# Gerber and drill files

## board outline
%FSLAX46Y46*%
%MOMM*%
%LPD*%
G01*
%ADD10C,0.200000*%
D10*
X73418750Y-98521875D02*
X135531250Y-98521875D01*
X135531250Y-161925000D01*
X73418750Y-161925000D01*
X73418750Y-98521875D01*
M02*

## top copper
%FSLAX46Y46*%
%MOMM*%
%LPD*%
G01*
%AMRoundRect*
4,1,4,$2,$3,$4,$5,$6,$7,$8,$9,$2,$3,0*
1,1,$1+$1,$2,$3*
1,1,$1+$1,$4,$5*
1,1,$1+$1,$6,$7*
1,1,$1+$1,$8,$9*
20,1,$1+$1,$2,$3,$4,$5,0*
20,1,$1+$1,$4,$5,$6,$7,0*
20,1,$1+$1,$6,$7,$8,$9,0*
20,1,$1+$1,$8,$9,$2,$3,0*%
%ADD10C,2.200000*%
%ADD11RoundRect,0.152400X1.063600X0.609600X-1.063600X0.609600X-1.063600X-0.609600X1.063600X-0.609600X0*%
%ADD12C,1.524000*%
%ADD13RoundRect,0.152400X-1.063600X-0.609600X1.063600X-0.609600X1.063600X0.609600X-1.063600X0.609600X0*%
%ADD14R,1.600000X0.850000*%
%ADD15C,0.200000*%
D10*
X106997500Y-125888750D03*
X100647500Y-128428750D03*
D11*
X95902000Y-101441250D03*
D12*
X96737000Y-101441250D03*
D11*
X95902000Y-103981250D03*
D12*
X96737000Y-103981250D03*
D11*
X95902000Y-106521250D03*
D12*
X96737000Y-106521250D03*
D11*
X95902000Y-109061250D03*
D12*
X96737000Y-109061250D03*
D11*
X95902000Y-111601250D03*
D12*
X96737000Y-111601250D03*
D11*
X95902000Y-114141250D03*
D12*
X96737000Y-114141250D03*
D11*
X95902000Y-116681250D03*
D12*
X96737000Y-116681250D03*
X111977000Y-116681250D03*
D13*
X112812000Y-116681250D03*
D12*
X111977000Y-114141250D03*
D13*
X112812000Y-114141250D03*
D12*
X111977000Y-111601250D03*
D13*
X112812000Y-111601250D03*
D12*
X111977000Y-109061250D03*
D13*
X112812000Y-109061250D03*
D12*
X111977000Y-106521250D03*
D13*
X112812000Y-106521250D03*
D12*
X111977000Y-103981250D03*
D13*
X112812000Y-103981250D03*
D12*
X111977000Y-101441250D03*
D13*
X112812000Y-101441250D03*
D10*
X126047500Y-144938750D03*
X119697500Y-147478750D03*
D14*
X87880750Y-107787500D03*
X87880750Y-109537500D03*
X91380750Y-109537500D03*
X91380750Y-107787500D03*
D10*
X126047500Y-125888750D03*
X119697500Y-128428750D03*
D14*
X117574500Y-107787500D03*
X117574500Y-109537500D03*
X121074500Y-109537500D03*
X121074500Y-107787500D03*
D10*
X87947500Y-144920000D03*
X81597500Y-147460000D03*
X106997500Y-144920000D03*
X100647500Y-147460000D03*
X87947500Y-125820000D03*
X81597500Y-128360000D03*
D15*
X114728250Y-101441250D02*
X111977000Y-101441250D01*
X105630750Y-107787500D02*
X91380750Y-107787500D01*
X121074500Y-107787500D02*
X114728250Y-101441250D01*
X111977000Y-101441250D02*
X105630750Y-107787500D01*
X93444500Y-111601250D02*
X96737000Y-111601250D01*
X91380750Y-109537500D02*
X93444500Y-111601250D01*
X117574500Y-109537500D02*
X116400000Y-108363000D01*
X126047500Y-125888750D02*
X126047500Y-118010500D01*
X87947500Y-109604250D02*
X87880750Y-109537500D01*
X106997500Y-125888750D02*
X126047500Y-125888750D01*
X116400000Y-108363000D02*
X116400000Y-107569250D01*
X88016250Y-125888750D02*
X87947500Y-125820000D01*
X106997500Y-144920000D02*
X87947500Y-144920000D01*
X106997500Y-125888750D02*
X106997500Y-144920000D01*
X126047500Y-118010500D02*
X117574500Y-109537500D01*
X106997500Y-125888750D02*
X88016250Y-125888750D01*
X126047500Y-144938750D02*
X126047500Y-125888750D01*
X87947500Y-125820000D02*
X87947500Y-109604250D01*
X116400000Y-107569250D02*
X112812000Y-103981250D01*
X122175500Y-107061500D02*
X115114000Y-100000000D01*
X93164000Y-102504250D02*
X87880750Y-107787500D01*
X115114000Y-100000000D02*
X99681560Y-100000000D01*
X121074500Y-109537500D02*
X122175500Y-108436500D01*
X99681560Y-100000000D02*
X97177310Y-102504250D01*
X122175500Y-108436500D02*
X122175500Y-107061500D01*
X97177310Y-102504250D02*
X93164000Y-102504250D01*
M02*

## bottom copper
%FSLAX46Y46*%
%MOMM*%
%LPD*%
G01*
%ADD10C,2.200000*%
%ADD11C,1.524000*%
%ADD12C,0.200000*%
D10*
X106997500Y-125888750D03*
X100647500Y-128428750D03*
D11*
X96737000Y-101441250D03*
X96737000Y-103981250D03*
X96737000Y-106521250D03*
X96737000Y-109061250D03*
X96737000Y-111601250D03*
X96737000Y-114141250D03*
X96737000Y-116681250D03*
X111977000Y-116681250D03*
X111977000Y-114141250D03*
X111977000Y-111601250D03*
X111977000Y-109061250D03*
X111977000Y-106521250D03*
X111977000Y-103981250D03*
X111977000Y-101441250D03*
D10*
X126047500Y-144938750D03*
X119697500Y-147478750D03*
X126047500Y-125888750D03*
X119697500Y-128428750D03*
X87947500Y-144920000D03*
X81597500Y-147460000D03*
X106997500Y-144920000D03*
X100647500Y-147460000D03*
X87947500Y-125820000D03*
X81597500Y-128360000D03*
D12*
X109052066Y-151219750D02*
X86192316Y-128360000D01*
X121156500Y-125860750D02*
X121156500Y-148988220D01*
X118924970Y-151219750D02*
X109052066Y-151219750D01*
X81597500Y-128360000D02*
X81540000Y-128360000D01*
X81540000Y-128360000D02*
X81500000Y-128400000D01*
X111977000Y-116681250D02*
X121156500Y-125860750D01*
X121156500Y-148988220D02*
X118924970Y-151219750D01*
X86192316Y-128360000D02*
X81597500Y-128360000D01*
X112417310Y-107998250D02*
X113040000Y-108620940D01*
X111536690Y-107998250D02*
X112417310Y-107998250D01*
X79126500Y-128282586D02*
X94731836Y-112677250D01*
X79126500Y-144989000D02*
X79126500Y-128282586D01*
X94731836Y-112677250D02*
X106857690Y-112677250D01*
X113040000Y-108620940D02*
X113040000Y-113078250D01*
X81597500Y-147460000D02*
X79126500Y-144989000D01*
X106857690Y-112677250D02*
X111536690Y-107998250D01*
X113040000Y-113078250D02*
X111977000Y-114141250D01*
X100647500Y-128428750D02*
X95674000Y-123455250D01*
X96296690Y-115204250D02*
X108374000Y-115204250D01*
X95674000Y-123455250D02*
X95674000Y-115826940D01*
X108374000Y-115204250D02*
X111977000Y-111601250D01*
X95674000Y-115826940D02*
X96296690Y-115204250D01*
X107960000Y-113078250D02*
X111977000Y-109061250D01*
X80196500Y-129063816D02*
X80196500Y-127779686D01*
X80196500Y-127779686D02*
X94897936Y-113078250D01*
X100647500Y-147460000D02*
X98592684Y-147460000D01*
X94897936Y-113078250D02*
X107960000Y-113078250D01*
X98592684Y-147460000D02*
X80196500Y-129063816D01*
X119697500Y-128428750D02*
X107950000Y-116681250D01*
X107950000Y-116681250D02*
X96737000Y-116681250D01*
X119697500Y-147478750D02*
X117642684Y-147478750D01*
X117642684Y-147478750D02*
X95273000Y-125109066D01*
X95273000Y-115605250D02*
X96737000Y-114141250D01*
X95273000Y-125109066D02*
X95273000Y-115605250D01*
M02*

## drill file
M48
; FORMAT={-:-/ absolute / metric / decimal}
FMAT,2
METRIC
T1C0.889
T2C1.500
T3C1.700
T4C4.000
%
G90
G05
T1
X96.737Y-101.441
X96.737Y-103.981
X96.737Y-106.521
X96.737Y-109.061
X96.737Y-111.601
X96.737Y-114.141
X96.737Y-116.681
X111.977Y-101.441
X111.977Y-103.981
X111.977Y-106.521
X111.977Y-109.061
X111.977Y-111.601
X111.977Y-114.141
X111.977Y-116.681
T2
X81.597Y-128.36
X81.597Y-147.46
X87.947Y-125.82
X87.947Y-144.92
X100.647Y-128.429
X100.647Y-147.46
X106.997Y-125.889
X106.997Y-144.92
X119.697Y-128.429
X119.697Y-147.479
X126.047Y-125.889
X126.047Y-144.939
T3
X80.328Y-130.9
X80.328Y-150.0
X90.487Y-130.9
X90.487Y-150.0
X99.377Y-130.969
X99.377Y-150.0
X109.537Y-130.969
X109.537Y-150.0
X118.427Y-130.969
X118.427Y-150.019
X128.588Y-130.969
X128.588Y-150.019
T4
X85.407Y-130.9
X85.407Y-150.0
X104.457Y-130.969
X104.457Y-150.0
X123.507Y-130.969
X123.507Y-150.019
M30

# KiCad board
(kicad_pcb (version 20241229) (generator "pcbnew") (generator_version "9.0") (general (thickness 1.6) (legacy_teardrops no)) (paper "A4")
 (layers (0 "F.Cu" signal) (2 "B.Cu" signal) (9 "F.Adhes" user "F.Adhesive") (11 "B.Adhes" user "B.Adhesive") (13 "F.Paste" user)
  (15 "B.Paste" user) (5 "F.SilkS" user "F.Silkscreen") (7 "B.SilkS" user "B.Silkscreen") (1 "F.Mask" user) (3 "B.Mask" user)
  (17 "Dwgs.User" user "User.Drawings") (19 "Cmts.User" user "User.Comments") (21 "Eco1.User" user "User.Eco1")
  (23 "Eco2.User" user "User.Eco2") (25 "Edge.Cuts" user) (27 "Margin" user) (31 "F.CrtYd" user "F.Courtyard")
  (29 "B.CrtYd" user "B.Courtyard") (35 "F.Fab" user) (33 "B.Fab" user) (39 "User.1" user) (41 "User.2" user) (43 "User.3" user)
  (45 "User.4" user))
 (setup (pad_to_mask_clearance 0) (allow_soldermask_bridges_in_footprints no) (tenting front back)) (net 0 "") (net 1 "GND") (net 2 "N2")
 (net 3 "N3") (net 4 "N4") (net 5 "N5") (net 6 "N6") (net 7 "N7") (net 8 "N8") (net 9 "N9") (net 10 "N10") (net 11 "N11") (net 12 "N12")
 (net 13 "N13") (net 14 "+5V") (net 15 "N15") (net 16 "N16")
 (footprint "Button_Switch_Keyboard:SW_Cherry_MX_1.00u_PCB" (layer "F.Cu") (at 106.9975 125.88875)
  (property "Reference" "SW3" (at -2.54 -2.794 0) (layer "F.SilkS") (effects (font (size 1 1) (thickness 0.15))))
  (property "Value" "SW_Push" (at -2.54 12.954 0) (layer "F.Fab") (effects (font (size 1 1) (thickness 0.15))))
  (pad "" np_thru_hole circle (at -7.62 5.08) (size 1.7 1.7) (drill 1.7) (layers "*.Cu" "*.Mask"))
  (pad "" np_thru_hole circle (at -2.54 5.08) (size 4 4) (drill 4) (layers "*.Cu" "*.Mask"))
  (pad "" np_thru_hole circle (at 2.54 5.08) (size 1.7 1.7) (drill 1.7) (layers "*.Cu" "*.Mask"))
  (pad "1" thru_hole circle (at 0 0) (size 2.2 2.2) (drill 1.5) (layers "*.Cu" "*.Mask") (remove_unused_layers no) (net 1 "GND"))
  (pad "2" thru_hole circle (at -6.35 2.54) (size 2.2 2.2) (drill 1.5) (layers "*.Cu" "*.Mask") (remove_unused_layers no) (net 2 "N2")))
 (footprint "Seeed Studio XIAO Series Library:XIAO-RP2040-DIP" (layer "F.Cu") (at 104.357 109.06125)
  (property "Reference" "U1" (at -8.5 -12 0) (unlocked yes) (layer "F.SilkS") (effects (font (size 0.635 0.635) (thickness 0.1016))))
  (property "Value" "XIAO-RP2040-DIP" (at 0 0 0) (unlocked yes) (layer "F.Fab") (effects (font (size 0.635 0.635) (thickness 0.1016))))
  (pad "1" smd roundrect (at -8.455 -7.62 180) (size 2.432 1.524) (layers "F.Cu" "F.Mask") (roundrect_rratio 0.1) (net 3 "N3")
   (thermal_bridge_angle 45))
  (pad "1" thru_hole circle (at -7.62 -7.62 180) (size 1.524 1.524) (drill 0.889) (layers "*.Cu" "*.Mask") (remove_unused_layers no)
   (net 3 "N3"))
  (pad "2" smd roundrect (at -8.455 -5.08 180) (size 2.432 1.524) (layers "F.Cu" "F.Mask") (roundrect_rratio 0.1) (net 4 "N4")
   (thermal_bridge_angle 45))
  (pad "2" thru_hole circle (at -7.62 -5.08 180) (size 1.524 1.524) (drill 0.889) (layers "*.Cu" "*.Mask") (remove_unused_layers no)
   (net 4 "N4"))
  (pad "3" smd roundrect (at -8.455 -2.54 180) (size 2.432 1.524) (layers "F.Cu" "F.Mask") (roundrect_rratio 0.1) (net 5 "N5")
   (thermal_bridge_angle 45))
  (pad "3" thru_hole circle (at -7.62 -2.54 180) (size 1.524 1.524) (drill 0.889) (layers "*.Cu" "*.Mask") (remove_unused_layers no)
   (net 5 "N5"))
  (pad "4" smd roundrect (at -8.455 0 180) (size 2.432 1.524) (layers "F.Cu" "F.Mask") (roundrect_rratio 0.1) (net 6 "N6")
   (thermal_bridge_angle 45))
  (pad "4" thru_hole circle (at -7.62 0 180) (size 1.524 1.524) (drill 0.889) (layers "*.Cu" "*.Mask") (remove_unused_layers no)
   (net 6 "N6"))
  (pad "5" smd roundrect (at -8.455 2.54 180) (size 2.432 1.524) (layers "F.Cu" "F.Mask") (roundrect_rratio 0.1) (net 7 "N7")
   (thermal_bridge_angle 45))
  (pad "5" thru_hole circle (at -7.62 2.54 180) (size 1.524 1.524) (drill 0.889) (layers "*.Cu" "*.Mask") (remove_unused_layers no)
   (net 7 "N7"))
  (pad "6" smd roundrect (at -8.455 5.08 180) (size 2.432 1.524) (layers "F.Cu" "F.Mask") (roundrect_rratio 0.1) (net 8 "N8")
   (thermal_bridge_angle 45))
  (pad "6" thru_hole circle (at -7.62 5.08 180) (size 1.524 1.524) (drill 0.889) (layers "*.Cu" "*.Mask") (remove_unused_layers no)
   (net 8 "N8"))
  (pad "7" smd roundrect (at -8.455 7.62 180) (size 2.432 1.524) (layers "F.Cu" "F.Mask") (roundrect_rratio 0.1) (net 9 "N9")
   (thermal_bridge_angle 45))
  (pad "7" thru_hole circle (at -7.62 7.62 180) (size 1.524 1.524) (drill 0.889) (layers "*.Cu" "*.Mask") (remove_unused_layers no)
   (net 9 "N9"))
  (pad "8" thru_hole circle (at 7.62 7.62) (size 1.524 1.524) (drill 0.889) (layers "*.Cu" "*.Mask") (remove_unused_layers no)
   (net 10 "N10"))
  (pad "8" smd roundrect (at 8.455 7.62) (size 2.432 1.524) (layers "F.Cu" "F.Mask") (roundrect_rratio 0.1) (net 10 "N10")
   (thermal_bridge_angle 45))
  (pad "9" thru_hole circle (at 7.62 5.08) (size 1.524 1.524) (drill 0.889) (layers "*.Cu" "*.Mask") (remove_unused_layers no)
   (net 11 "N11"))
  (pad "9" smd roundrect (at 8.455 5.08) (size 2.432 1.524) (layers "F.Cu" "F.Mask") (roundrect_rratio 0.1) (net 11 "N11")
   (thermal_bridge_angle 45))
  (pad "10" thru_hole circle (at 7.62 2.54) (size 1.524 1.524) (drill 0.889) (layers "*.Cu" "*.Mask") (remove_unused_layers no) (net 2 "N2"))
  (pad "10" smd roundrect (at 8.455 2.54) (size 2.432 1.524) (layers "F.Cu" "F.Mask") (roundrect_rratio 0.1) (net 2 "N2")
   (thermal_bridge_angle 45))
  (pad "11" thru_hole circle (at 7.62 0) (size 1.524 1.524) (drill 0.889) (layers "*.Cu" "*.Mask") (remove_unused_layers no) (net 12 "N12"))
  (pad "11" smd roundrect (at 8.455 0) (size 2.432 1.524) (layers "F.Cu" "F.Mask") (roundrect_rratio 0.1) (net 12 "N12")
   (thermal_bridge_angle 45))
  (pad "12" thru_hole circle (at 7.62 -2.54) (size 1.524 1.524) (drill 0.889) (layers "*.Cu" "*.Mask") (remove_unused_layers no)
   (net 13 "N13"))
  (pad "12" smd roundrect (at 8.455 -2.54) (size 2.432 1.524) (layers "F.Cu" "F.Mask") (roundrect_rratio 0.1) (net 13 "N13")
   (thermal_bridge_angle 45))
  (pad "13" thru_hole circle (at 7.62 -5.08) (size 1.524 1.524) (drill 0.889) (layers "*.Cu" "*.Mask") (remove_unused_layers no)
   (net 1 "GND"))
  (pad "13" smd roundrect (at 8.455 -5.08) (size 2.432 1.524) (layers "F.Cu" "F.Mask") (roundrect_rratio 0.1) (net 1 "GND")
   (thermal_bridge_angle 45))
  (pad "14" thru_hole circle (at 7.62 -7.62) (size 1.524 1.524) (drill 0.889) (layers "*.Cu" "*.Mask") (remove_unused_layers no)
   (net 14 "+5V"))
  (pad "14" smd roundrect (at 8.455 -7.62) (size 2.432 1.524) (layers "F.Cu" "F.Mask") (roundrect_rratio 0.1) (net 14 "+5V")
   (thermal_bridge_angle 45)))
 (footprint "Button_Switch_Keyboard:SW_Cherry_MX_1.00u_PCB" (layer "F.Cu") (at 126.0475 144.93875)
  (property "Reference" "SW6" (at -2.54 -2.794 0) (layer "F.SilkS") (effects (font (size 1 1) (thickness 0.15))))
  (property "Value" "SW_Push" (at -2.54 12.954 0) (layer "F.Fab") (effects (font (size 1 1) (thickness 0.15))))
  (pad "" np_thru_hole circle (at -7.62 5.08) (size 1.7 1.7) (drill 1.7) (layers "*.Cu" "*.Mask"))
  (pad "" np_thru_hole circle (at -2.54 5.08) (size 4 4) (drill 4) (layers "*.Cu" "*.Mask"))
  (pad "" np_thru_hole circle (at 2.54 5.08) (size 1.7 1.7) (drill 1.7) (layers "*.Cu" "*.Mask"))
  (pad "1" thru_hole circle (at 0 0) (size 2.2 2.2) (drill 1.5) (layers "*.Cu" "*.Mask") (remove_unused_layers no) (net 1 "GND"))
  (pad "2" thru_hole circle (at -6.35 2.54) (size 2.2 2.2) (drill 1.5) (layers "*.Cu" "*.Mask") (remove_unused_layers no) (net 8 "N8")))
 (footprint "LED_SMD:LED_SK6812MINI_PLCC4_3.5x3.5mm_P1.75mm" (layer "F.Cu") (at 89.63075 108.6625)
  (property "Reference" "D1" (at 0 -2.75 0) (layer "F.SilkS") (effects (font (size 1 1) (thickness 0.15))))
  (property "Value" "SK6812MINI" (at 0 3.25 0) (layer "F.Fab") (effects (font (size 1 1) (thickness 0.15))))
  (pad "1" smd rect (at -1.75 -0.875) (size 1.6 0.85) (layers "F.Cu" "F.Mask" "F.Paste") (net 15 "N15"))
  (pad "2" smd rect (at -1.75 0.875) (size 1.6 0.85) (layers "F.Cu" "F.Mask" "F.Paste") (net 1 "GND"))
  (pad "3" smd rect (at 1.75 0.875) (size 1.6 0.85) (layers "F.Cu" "F.Mask" "F.Paste") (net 7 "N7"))
  (pad "4" smd rect (at 1.75 -0.875) (size 1.6 0.85) (layers "F.Cu" "F.Mask" "F.Paste") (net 14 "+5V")))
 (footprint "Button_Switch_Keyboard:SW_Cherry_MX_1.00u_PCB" (layer "F.Cu") (at 126.0475 125.88875)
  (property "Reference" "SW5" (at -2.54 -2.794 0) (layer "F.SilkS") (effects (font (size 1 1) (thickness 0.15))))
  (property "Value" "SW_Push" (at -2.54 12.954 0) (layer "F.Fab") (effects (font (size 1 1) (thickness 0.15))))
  (pad "" np_thru_hole circle (at -7.62 5.08) (size 1.7 1.7) (drill 1.7) (layers "*.Cu" "*.Mask"))
  (pad "" np_thru_hole circle (at -2.54 5.08) (size 4 4) (drill 4) (layers "*.Cu" "*.Mask"))
  (pad "" np_thru_hole circle (at 2.54 5.08) (size 1.7 1.7) (drill 1.7) (layers "*.Cu" "*.Mask"))
  (pad "1" thru_hole circle (at 0 0) (size 2.2 2.2) (drill 1.5) (layers "*.Cu" "*.Mask") (remove_unused_layers no) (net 1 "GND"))
  (pad "2" thru_hole circle (at -6.35 2.54) (size 2.2 2.2) (drill 1.5) (layers "*.Cu" "*.Mask") (remove_unused_layers no) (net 9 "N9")))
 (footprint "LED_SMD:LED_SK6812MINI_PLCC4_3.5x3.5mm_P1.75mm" (layer "F.Cu") (at 119.3245 108.6625)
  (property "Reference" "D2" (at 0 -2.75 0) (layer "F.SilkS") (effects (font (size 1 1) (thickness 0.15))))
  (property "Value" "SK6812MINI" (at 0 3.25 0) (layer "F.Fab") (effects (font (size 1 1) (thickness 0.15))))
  (pad "1" smd rect (at -1.75 -0.875) (size 1.6 0.85) (layers "F.Cu" "F.Mask" "F.Paste") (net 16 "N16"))
  (pad "2" smd rect (at -1.75 0.875) (size 1.6 0.85) (layers "F.Cu" "F.Mask" "F.Paste") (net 1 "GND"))
  (pad "3" smd rect (at 1.75 0.875) (size 1.6 0.85) (layers "F.Cu" "F.Mask" "F.Paste") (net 15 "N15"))
  (pad "4" smd rect (at 1.75 -0.875) (size 1.6 0.85) (layers "F.Cu" "F.Mask" "F.Paste") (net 14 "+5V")))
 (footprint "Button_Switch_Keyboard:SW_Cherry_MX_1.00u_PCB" (layer "F.Cu") (at 87.9475 144.92)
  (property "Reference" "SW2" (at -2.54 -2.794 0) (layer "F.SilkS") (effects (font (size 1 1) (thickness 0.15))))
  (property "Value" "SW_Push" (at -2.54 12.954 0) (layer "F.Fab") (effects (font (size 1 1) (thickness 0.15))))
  (pad "" np_thru_hole circle (at -7.62 5.08) (size 1.7 1.7) (drill 1.7) (layers "*.Cu" "*.Mask"))
  (pad "" np_thru_hole circle (at -2.54 5.08) (size 4 4) (drill 4) (layers "*.Cu" "*.Mask"))
  (pad "" np_thru_hole circle (at 2.54 5.08) (size 1.7 1.7) (drill 1.7) (layers "*.Cu" "*.Mask"))
  (pad "1" thru_hole circle (at 0 0) (size 2.2 2.2) (drill 1.5) (layers "*.Cu" "*.Mask") (remove_unused_layers no) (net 1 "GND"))
  (pad "2" thru_hole circle (at -6.35 2.54) (size 2.2 2.2) (drill 1.5) (layers "*.Cu" "*.Mask") (remove_unused_layers no) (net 11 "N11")))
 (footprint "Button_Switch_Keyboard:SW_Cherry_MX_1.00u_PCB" (layer "F.Cu") (at 106.9975 144.92)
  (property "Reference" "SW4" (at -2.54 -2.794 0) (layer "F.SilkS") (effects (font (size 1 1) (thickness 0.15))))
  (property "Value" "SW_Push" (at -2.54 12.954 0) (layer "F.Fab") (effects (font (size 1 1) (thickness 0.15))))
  (pad "" np_thru_hole circle (at -7.62 5.08) (size 1.7 1.7) (drill 1.7) (layers "*.Cu" "*.Mask"))
  (pad "" np_thru_hole circle (at -2.54 5.08) (size 4 4) (drill 4) (layers "*.Cu" "*.Mask"))
  (pad "" np_thru_hole circle (at 2.54 5.08) (size 1.7 1.7) (drill 1.7) (layers "*.Cu" "*.Mask"))
  (pad "1" thru_hole circle (at 0 0) (size 2.2 2.2) (drill 1.5) (layers "*.Cu" "*.Mask") (remove_unused_layers no) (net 1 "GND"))
  (pad "2" thru_hole circle (at -6.35 2.54) (size 2.2 2.2) (drill 1.5) (layers "*.Cu" "*.Mask") (remove_unused_layers no) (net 12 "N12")))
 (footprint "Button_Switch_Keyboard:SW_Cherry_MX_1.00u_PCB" (layer "F.Cu") (at 87.9475 125.82)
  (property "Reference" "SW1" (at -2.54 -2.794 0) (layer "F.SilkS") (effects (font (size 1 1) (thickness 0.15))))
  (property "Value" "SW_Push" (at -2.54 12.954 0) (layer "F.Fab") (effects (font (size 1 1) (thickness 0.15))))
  (pad "" np_thru_hole circle (at -7.62 5.08) (size 1.7 1.7) (drill 1.7) (layers "*.Cu" "*.Mask"))
  (pad "" np_thru_hole circle (at -2.54 5.08) (size 4 4) (drill 4) (layers "*.Cu" "*.Mask"))
  (pad "" np_thru_hole circle (at 2.54 5.08) (size 1.7 1.7) (drill 1.7) (layers "*.Cu" "*.Mask"))
  (pad "1" thru_hole circle (at 0 0) (size 2.2 2.2) (drill 1.5) (layers "*.Cu" "*.Mask") (remove_unused_layers no) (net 1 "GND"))
  (pad "2" thru_hole circle (at -6.35 2.54) (size 2.2 2.2) (drill 1.5) (layers "*.Cu" "*.Mask") (remove_unused_layers no) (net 10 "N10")))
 (gr_rect (start 73.41875 98.521875) (end 135.53125 161.925) (stroke (width 0.2) (type solid)) (fill no) (layer "Edge.Cuts"))
 (segment (start 114.72825 101.44125) (end 111.977 101.44125) (width 0.2) (layer "F.Cu") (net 14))
 (segment (start 105.63075 107.7875) (end 91.38075 107.7875) (width 0.2) (layer "F.Cu") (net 14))
 (segment (start 121.0745 107.7875) (end 114.72825 101.44125) (width 0.2) (layer "F.Cu") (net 14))
 (segment (start 111.977 101.44125) (end 105.63075 107.7875) (width 0.2) (layer "F.Cu") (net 14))
 (segment (start 93.4445 111.60125) (end 96.737 111.60125) (width 0.2) (layer "F.Cu") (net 7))
 (segment (start 91.38075 109.5375) (end 93.4445 111.60125) (width 0.2) (layer "F.Cu") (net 7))
 (segment (start 117.5745 109.5375) (end 116.4 108.363) (width 0.2) (layer "F.Cu") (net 1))
 (segment (start 126.0475 125.88875) (end 126.0475 118.0105) (width 0.2) (layer "F.Cu") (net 1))
 (segment (start 87.9475 109.60425) (end 87.88075 109.5375) (width 0.2) (layer "F.Cu") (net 1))
 (segment (start 106.9975 125.88875) (end 126.0475 125.88875) (width 0.2) (layer "F.Cu") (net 1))
 (segment (start 116.4 108.363) (end 116.4 107.56925) (width 0.2) (layer "F.Cu") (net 1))
 (segment (start 88.01625 125.88875) (end 87.9475 125.82) (width 0.2) (layer "F.Cu") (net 1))
 (segment (start 106.9975 144.92) (end 87.9475 144.92) (width 0.2) (layer "F.Cu") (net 1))
 (segment (start 106.9975 125.88875) (end 106.9975 144.92) (width 0.2) (layer "F.Cu") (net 1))
 (segment (start 126.0475 118.0105) (end 117.5745 109.5375) (width 0.2) (layer "F.Cu") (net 1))
 (segment (start 106.9975 125.88875) (end 88.01625 125.88875) (width 0.2) (layer "F.Cu") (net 1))
 (segment (start 126.0475 144.93875) (end 126.0475 125.88875) (width 0.2) (layer "F.Cu") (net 1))
 (segment (start 87.9475 125.82) (end 87.9475 109.60425) (width 0.2) (layer "F.Cu") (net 1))
 (segment (start 116.4 107.56925) (end 112.812 103.98125) (width 0.2) (layer "F.Cu") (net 1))
 (segment (start 122.1755 107.0615) (end 115.114 100) (width 0.2) (layer "F.Cu") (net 15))
 (segment (start 93.164 102.50425) (end 87.88075 107.7875) (width 0.2) (layer "F.Cu") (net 15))
 (segment (start 115.114 100) (end 99.68156 100) (width 0.2) (layer "F.Cu") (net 15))
 (segment (start 121.0745 109.5375) (end 122.1755 108.4365) (width 0.2) (layer "F.Cu") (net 15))
 (segment (start 99.68156 100) (end 97.17731 102.50425) (width 0.2) (layer "F.Cu") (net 15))
 (segment (start 122.1755 108.4365) (end 122.1755 107.0615) (width 0.2) (layer "F.Cu") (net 15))
 (segment (start 97.17731 102.50425) (end 93.164 102.50425) (width 0.2) (layer "F.Cu") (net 15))
 (segment (start 109.052066 151.21975) (end 86.192316 128.36) (width 0.2) (layer "B.Cu") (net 10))
 (segment (start 121.1565 125.86075) (end 121.1565 148.98822) (width 0.2) (layer "B.Cu") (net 10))
 (segment (start 118.92497 151.21975) (end 109.052066 151.21975) (width 0.2) (layer "B.Cu") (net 10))
 (segment (start 81.5975 128.36) (end 81.54 128.36) (width 0.2) (layer "B.Cu") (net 10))
 (segment (start 81.54 128.36) (end 81.5 128.4) (width 0.2) (layer "B.Cu") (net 10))
 (segment (start 111.977 116.68125) (end 121.1565 125.86075) (width 0.2) (layer "B.Cu") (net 10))
 (segment (start 121.1565 148.98822) (end 118.92497 151.21975) (width 0.2) (layer "B.Cu") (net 10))
 (segment (start 86.192316 128.36) (end 81.5975 128.36) (width 0.2) (layer "B.Cu") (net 10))
 (segment (start 112.41731 107.99825) (end 113.04 108.62094) (width 0.2) (layer "B.Cu") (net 11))
 (segment (start 111.53669 107.99825) (end 112.41731 107.99825) (width 0.2) (layer "B.Cu") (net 11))
 (segment (start 79.1265 128.282586) (end 94.731836 112.67725) (width 0.2) (layer "B.Cu") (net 11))
 (segment (start 79.1265 144.989) (end 79.1265 128.282586) (width 0.2) (layer "B.Cu") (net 11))
 (segment (start 94.731836 112.67725) (end 106.85769 112.67725) (width 0.2) (layer "B.Cu") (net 11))
 (segment (start 113.04 108.62094) (end 113.04 113.07825) (width 0.2) (layer "B.Cu") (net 11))
 (segment (start 81.5975 147.46) (end 79.1265 144.989) (width 0.2) (layer "B.Cu") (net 11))
 (segment (start 106.85769 112.67725) (end 111.53669 107.99825) (width 0.2) (layer "B.Cu") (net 11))
 (segment (start 113.04 113.07825) (end 111.977 114.14125) (width 0.2) (layer "B.Cu") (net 11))
 (segment (start 100.6475 128.42875) (end 95.674 123.45525) (width 0.2) (layer "B.Cu") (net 2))
 (segment (start 96.29669 115.20425) (end 108.374 115.20425) (width 0.2) (layer "B.Cu") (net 2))
 (segment (start 95.674 123.45525) (end 95.674 115.82694) (width 0.2) (layer "B.Cu") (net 2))
 (segment (start 108.374 115.20425) (end 111.977 111.60125) (width 0.2) (layer "B.Cu") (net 2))
 (segment (start 95.674 115.82694) (end 96.29669 115.20425) (width 0.2) (layer "B.Cu") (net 2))
 (segment (start 107.96 113.07825) (end 111.977 109.06125) (width 0.2) (layer "B.Cu") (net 12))
 (segment (start 80.1965 129.063816) (end 80.1965 127.779686) (width 0.2) (layer "B.Cu") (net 12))
 (segment (start 80.1965 127.779686) (end 94.897936 113.07825) (width 0.2) (layer "B.Cu") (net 12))
 (segment (start 100.6475 147.46) (end 98.592684 147.46) (width 0.2) (layer "B.Cu") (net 12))
 (segment (start 94.897936 113.07825) (end 107.96 113.07825) (width 0.2) (layer "B.Cu") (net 12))
 (segment (start 98.592684 147.46) (end 80.1965 129.063816) (width 0.2) (layer "B.Cu") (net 12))
 (segment (start 119.6975 128.42875) (end 107.95 116.68125) (width 0.2) (layer "B.Cu") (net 9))
 (segment (start 107.95 116.68125) (end 96.737 116.68125) (width 0.2) (layer "B.Cu") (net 9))
 (segment (start 119.6975 147.47875) (end 117.642684 147.47875) (width 0.2) (layer "B.Cu") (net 8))
 (segment (start 117.642684 147.47875) (end 95.273 125.109066) (width 0.2) (layer "B.Cu") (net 8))
 (segment (start 95.273 115.60525) (end 96.737 114.14125) (width 0.2) (layer "B.Cu") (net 8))
 (segment (start 95.273 125.109066) (end 95.273 115.60525) (width 0.2) (layer "B.Cu") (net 8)))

